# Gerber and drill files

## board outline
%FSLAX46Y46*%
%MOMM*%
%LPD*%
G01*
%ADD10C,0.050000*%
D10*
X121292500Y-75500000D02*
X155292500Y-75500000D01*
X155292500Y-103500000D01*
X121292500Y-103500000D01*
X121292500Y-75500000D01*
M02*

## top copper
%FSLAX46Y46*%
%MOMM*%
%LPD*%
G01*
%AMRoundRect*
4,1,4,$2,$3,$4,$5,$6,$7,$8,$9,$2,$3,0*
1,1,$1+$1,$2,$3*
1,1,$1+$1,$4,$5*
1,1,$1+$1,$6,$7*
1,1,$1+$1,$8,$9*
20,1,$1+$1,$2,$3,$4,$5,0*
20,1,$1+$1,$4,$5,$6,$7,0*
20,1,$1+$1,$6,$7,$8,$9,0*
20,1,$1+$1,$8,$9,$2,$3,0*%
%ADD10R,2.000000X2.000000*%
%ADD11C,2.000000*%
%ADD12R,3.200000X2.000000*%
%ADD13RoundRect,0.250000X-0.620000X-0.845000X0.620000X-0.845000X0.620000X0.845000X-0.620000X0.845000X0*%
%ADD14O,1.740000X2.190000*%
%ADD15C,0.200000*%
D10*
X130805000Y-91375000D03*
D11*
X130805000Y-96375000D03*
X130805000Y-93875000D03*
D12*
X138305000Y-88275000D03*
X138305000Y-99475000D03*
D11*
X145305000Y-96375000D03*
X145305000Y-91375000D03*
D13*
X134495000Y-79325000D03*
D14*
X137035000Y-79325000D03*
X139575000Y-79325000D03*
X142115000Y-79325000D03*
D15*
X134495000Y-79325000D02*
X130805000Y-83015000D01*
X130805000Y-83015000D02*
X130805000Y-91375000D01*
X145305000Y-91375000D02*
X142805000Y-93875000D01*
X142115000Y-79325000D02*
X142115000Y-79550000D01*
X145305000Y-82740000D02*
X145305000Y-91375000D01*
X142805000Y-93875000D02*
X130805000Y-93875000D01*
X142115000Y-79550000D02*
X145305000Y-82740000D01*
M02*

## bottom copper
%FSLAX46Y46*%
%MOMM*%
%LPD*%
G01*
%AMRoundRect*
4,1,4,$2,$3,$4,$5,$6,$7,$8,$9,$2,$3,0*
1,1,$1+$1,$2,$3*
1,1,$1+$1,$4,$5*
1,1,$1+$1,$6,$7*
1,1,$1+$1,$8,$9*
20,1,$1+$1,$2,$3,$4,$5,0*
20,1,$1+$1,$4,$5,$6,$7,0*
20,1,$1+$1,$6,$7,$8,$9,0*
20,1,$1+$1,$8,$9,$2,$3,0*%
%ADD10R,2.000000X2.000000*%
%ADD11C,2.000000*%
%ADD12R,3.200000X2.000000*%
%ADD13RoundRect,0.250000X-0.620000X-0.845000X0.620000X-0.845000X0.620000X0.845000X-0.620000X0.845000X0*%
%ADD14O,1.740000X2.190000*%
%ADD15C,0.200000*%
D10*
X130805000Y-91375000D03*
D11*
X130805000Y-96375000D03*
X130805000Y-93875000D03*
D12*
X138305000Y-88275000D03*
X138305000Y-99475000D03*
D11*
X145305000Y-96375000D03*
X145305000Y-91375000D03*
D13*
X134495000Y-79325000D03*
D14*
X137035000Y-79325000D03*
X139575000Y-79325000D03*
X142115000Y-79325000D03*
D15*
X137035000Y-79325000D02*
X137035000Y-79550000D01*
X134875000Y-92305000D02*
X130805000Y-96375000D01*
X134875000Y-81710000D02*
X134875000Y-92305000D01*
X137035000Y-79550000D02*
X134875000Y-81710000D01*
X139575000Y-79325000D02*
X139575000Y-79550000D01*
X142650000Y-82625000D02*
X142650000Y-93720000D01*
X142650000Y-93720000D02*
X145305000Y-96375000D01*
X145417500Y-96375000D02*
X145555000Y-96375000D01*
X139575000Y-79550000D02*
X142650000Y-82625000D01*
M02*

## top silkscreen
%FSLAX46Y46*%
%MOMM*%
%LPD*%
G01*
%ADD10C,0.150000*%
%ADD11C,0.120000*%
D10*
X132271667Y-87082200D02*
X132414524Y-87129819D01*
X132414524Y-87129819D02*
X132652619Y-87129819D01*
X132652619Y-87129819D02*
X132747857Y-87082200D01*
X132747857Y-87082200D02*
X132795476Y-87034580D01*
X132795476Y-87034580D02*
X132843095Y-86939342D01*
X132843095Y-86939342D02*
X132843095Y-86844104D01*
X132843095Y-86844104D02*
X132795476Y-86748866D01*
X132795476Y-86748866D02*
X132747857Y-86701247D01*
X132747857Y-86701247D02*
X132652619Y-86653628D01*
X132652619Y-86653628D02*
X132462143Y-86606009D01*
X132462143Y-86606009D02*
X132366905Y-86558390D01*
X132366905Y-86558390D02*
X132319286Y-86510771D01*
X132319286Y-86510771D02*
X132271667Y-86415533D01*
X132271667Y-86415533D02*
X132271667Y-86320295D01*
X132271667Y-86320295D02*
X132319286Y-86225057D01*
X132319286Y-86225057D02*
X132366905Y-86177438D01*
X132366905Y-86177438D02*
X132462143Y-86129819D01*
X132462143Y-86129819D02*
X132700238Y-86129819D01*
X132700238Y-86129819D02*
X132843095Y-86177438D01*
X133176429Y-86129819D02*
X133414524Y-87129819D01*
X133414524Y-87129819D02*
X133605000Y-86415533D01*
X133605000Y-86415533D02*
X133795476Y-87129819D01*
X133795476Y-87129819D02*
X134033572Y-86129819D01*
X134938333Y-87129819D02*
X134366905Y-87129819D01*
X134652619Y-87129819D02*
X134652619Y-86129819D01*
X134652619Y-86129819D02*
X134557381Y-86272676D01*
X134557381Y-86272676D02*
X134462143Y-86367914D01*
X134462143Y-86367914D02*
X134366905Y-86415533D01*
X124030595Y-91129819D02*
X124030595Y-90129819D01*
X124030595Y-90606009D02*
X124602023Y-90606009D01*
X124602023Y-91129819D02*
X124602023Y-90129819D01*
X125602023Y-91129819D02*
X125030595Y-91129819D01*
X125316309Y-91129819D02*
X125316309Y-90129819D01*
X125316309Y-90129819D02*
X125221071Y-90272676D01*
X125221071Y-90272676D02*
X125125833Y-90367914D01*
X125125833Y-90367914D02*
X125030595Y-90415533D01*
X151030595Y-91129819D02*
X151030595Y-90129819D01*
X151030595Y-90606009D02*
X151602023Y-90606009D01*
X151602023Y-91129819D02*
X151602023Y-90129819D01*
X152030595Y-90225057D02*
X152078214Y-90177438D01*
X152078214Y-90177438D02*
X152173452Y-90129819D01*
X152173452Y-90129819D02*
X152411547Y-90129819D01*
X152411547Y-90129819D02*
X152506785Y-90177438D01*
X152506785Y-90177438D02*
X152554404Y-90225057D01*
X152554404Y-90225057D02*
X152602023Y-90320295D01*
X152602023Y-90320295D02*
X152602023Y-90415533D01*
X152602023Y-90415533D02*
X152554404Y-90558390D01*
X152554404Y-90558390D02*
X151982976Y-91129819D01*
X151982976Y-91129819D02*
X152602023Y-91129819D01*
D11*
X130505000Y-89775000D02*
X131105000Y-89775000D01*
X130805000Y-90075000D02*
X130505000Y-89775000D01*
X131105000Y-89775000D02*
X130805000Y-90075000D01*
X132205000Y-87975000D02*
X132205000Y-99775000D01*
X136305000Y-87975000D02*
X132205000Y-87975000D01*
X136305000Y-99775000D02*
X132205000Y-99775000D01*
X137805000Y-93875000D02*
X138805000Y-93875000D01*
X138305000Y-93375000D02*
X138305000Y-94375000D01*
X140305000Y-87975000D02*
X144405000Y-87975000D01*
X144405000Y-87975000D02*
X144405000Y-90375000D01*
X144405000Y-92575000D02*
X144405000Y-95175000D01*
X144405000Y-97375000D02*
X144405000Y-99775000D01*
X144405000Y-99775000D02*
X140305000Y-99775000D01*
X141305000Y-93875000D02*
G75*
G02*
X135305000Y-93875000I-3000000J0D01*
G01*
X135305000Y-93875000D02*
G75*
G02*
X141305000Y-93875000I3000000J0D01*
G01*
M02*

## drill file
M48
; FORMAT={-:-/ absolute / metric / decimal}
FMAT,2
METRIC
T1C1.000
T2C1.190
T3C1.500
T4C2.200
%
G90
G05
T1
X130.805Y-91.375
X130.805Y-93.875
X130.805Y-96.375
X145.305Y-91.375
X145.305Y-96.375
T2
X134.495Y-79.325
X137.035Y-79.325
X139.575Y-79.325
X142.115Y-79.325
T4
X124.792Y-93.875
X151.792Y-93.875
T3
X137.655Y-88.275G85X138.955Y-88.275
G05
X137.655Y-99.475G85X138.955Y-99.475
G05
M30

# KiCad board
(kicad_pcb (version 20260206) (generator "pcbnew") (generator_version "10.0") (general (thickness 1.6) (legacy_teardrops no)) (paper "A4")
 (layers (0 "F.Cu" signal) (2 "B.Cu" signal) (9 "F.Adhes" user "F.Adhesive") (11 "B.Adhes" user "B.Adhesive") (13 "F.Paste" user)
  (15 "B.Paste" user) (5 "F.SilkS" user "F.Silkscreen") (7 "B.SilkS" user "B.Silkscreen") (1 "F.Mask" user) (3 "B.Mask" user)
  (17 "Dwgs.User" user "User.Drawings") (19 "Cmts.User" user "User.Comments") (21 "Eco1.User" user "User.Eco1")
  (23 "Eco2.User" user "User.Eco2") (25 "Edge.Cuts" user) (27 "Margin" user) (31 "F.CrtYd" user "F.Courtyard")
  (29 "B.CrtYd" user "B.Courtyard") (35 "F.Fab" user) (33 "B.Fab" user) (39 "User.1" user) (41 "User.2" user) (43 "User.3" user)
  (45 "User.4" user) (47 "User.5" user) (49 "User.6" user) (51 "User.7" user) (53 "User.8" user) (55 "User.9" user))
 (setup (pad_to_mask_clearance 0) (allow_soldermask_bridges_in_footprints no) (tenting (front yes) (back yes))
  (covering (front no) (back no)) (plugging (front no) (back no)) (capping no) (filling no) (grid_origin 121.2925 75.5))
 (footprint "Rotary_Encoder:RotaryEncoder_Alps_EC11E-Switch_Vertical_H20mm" (layer "F.Cu") (at 130.805 91.375)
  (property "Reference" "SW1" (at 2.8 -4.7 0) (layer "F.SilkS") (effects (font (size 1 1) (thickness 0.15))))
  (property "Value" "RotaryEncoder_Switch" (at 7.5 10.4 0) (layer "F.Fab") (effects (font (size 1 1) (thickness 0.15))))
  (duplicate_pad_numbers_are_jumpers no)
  (fp_line (start -0.3 -1.6) (end 0.3 -1.6) (stroke (width 0.12) (type solid)) (layer "F.SilkS"))
  (fp_line (start 0 -1.3) (end -0.3 -1.6) (stroke (width 0.12) (type solid)) (layer "F.SilkS"))
  (fp_line (start 0.3 -1.6) (end 0 -1.3) (stroke (width 0.12) (type solid)) (layer "F.SilkS"))
  (fp_line (start 1.4 -3.4) (end 1.4 8.4) (stroke (width 0.12) (type solid)) (layer "F.SilkS"))
  (fp_line (start 5.5 -3.4) (end 1.4 -3.4) (stroke (width 0.12) (type solid)) (layer "F.SilkS"))
  (fp_line (start 5.5 8.4) (end 1.4 8.4) (stroke (width 0.12) (type solid)) (layer "F.SilkS"))
  (fp_line (start 7 2.5) (end 8 2.5) (stroke (width 0.12) (type solid)) (layer "F.SilkS"))
  (fp_line (start 7.5 2) (end 7.5 3) (stroke (width 0.12) (type solid)) (layer "F.SilkS"))
  (fp_line (start 9.5 -3.4) (end 13.6 -3.4) (stroke (width 0.12) (type solid)) (layer "F.SilkS"))
  (fp_line (start 13.6 -3.4) (end 13.6 -1) (stroke (width 0.12) (type solid)) (layer "F.SilkS"))
  (fp_line (start 13.6 1.2) (end 13.6 3.8) (stroke (width 0.12) (type solid)) (layer "F.SilkS"))
  (fp_line (start 13.6 6) (end 13.6 8.4) (stroke (width 0.12) (type solid)) (layer "F.SilkS"))
  (fp_line (start 13.6 8.4) (end 9.5 8.4) (stroke (width 0.12) (type solid)) (layer "F.SilkS"))
  (fp_circle (center 7.5 2.5) (end 10.5 2.5) (stroke (width 0.12) (type solid)) (fill no) (layer "F.SilkS"))
  (pad "A" thru_hole rect (at 0 0) (size 2 2) (drill 1) (layers "*.Cu" "*.Mask") (remove_unused_layers no) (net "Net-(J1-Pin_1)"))
  (pad "B" thru_hole circle (at 0 5) (size 2 2) (drill 1) (layers "*.Cu" "*.Mask") (remove_unused_layers no) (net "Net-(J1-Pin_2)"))
  (pad "C" thru_hole circle (at 0 2.5) (size 2 2) (drill 1) (layers "*.Cu" "*.Mask") (remove_unused_layers no) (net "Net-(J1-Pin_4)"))
  (pad "MP" thru_hole rect (at 7.5 -3.1) (size 3.2 2) (drill oval 2.8 1.5) (layers "*.Cu" "*.Mask") (remove_unused_layers no))
  (pad "MP" thru_hole rect (at 7.5 8.1) (size 3.2 2) (drill oval 2.8 1.5) (layers "*.Cu" "*.Mask") (remove_unused_layers no))
  (pad "S1" thru_hole circle (at 14.5 5) (size 2 2) (drill 1) (layers "*.Cu" "*.Mask") (remove_unused_layers no) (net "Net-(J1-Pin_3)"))
  (pad "S2" thru_hole circle (at 14.5 0) (size 2 2) (drill 1) (layers "*.Cu" "*.Mask") (remove_unused_layers no) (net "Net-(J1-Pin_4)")))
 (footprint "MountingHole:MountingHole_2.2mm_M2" (layer "F.Cu") (at 124.7925 93.875)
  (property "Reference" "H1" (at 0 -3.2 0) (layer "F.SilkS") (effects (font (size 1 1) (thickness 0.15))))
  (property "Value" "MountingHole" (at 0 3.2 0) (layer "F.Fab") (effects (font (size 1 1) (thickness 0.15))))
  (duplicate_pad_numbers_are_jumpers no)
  (pad "" np_thru_hole circle (at 0 0) (size 2.2 2.2) (drill 2.2) (layers "*.Cu" "*.Mask")))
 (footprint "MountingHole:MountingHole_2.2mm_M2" (layer "F.Cu") (at 151.7925 93.875)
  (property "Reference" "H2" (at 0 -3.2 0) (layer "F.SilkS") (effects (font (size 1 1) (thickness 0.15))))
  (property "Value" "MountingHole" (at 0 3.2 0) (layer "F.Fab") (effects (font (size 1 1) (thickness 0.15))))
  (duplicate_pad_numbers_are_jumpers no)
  (pad "" np_thru_hole circle (at 0 0) (size 2.2 2.2) (drill 2.2) (layers "*.Cu" "*.Mask")))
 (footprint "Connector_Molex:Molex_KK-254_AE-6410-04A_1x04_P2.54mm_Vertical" (layer "B.Cu") (at 134.495 79.325)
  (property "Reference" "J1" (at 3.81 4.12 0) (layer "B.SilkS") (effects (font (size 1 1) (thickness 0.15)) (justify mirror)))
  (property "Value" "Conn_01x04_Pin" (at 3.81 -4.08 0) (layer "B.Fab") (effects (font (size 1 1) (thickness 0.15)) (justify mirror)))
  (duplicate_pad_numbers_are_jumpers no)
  (pad "1" thru_hole roundrect (at 0 0) (size 1.74 2.19) (drill 1.19) (layers "*.Cu" "*.Mask") (remove_unused_layers no)
   (roundrect_rratio 0.1436781609) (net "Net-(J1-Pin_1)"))
  (pad "2" thru_hole oval (at 2.54 0) (size 1.74 2.19) (drill 1.19) (layers "*.Cu" "*.Mask") (remove_unused_layers no)
   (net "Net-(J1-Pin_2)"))
  (pad "3" thru_hole oval (at 5.08 0) (size 1.74 2.19) (drill 1.19) (layers "*.Cu" "*.Mask") (remove_unused_layers no)
   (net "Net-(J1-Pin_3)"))
  (pad "4" thru_hole oval (at 7.62 0) (size 1.74 2.19) (drill 1.19) (layers "*.Cu" "*.Mask") (remove_unused_layers no)
   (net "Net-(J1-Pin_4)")))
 (gr_rect (start 121.2925 75.5) (end 155.2925 103.5) (stroke (width 0.05) (type default)) (fill no) (layer "Edge.Cuts"))
 (segment (start 134.495 79.325) (end 130.805 83.015) (width 0.2) (layer "F.Cu") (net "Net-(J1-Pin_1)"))
 (segment (start 130.805 83.015) (end 130.805 91.375) (width 0.2) (layer "F.Cu") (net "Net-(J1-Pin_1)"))
 (segment (start 137.035 79.325) (end 137.035 79.55) (width 0.2) (layer "B.Cu") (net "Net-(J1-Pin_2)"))
 (segment (start 134.875 92.305) (end 130.805 96.375) (width 0.2) (layer "B.Cu") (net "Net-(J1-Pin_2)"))
 (segment (start 134.875 81.71) (end 134.875 92.305) (width 0.2) (layer "B.Cu") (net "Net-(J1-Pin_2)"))
 (segment (start 137.035 79.55) (end 134.875 81.71) (width 0.2) (layer "B.Cu") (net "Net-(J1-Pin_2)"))
 (segment (start 145.305 91.375) (end 142.805 93.875) (width 0.2) (layer "F.Cu") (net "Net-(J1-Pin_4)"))
 (segment (start 142.115 79.325) (end 142.115 79.55) (width 0.2) (layer "F.Cu") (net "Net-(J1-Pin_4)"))
 (segment (start 145.305 82.74) (end 145.305 91.375) (width 0.2) (layer "F.Cu") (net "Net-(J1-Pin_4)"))
 (segment (start 142.805 93.875) (end 130.805 93.875) (width 0.2) (layer "F.Cu") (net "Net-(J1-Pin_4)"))
 (segment (start 142.115 79.55) (end 145.305 82.74) (width 0.2) (layer "F.Cu") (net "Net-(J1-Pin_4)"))
 (segment (start 139.575 79.325) (end 139.575 79.55) (width 0.2) (layer "B.Cu") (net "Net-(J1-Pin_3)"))
 (segment (start 142.65 82.625) (end 142.65 93.72) (width 0.2) (layer "B.Cu") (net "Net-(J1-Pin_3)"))
 (segment (start 142.65 93.72) (end 145.305 96.375) (width 0.2) (layer "B.Cu") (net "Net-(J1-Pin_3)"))
 (segment (start 145.4175 96.375) (end 145.555 96.375) (width 0.2) (layer "B.Cu") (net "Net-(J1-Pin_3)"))
 (segment (start 139.575 79.55) (end 142.65 82.625) (width 0.2) (layer "B.Cu") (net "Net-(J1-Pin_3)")))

